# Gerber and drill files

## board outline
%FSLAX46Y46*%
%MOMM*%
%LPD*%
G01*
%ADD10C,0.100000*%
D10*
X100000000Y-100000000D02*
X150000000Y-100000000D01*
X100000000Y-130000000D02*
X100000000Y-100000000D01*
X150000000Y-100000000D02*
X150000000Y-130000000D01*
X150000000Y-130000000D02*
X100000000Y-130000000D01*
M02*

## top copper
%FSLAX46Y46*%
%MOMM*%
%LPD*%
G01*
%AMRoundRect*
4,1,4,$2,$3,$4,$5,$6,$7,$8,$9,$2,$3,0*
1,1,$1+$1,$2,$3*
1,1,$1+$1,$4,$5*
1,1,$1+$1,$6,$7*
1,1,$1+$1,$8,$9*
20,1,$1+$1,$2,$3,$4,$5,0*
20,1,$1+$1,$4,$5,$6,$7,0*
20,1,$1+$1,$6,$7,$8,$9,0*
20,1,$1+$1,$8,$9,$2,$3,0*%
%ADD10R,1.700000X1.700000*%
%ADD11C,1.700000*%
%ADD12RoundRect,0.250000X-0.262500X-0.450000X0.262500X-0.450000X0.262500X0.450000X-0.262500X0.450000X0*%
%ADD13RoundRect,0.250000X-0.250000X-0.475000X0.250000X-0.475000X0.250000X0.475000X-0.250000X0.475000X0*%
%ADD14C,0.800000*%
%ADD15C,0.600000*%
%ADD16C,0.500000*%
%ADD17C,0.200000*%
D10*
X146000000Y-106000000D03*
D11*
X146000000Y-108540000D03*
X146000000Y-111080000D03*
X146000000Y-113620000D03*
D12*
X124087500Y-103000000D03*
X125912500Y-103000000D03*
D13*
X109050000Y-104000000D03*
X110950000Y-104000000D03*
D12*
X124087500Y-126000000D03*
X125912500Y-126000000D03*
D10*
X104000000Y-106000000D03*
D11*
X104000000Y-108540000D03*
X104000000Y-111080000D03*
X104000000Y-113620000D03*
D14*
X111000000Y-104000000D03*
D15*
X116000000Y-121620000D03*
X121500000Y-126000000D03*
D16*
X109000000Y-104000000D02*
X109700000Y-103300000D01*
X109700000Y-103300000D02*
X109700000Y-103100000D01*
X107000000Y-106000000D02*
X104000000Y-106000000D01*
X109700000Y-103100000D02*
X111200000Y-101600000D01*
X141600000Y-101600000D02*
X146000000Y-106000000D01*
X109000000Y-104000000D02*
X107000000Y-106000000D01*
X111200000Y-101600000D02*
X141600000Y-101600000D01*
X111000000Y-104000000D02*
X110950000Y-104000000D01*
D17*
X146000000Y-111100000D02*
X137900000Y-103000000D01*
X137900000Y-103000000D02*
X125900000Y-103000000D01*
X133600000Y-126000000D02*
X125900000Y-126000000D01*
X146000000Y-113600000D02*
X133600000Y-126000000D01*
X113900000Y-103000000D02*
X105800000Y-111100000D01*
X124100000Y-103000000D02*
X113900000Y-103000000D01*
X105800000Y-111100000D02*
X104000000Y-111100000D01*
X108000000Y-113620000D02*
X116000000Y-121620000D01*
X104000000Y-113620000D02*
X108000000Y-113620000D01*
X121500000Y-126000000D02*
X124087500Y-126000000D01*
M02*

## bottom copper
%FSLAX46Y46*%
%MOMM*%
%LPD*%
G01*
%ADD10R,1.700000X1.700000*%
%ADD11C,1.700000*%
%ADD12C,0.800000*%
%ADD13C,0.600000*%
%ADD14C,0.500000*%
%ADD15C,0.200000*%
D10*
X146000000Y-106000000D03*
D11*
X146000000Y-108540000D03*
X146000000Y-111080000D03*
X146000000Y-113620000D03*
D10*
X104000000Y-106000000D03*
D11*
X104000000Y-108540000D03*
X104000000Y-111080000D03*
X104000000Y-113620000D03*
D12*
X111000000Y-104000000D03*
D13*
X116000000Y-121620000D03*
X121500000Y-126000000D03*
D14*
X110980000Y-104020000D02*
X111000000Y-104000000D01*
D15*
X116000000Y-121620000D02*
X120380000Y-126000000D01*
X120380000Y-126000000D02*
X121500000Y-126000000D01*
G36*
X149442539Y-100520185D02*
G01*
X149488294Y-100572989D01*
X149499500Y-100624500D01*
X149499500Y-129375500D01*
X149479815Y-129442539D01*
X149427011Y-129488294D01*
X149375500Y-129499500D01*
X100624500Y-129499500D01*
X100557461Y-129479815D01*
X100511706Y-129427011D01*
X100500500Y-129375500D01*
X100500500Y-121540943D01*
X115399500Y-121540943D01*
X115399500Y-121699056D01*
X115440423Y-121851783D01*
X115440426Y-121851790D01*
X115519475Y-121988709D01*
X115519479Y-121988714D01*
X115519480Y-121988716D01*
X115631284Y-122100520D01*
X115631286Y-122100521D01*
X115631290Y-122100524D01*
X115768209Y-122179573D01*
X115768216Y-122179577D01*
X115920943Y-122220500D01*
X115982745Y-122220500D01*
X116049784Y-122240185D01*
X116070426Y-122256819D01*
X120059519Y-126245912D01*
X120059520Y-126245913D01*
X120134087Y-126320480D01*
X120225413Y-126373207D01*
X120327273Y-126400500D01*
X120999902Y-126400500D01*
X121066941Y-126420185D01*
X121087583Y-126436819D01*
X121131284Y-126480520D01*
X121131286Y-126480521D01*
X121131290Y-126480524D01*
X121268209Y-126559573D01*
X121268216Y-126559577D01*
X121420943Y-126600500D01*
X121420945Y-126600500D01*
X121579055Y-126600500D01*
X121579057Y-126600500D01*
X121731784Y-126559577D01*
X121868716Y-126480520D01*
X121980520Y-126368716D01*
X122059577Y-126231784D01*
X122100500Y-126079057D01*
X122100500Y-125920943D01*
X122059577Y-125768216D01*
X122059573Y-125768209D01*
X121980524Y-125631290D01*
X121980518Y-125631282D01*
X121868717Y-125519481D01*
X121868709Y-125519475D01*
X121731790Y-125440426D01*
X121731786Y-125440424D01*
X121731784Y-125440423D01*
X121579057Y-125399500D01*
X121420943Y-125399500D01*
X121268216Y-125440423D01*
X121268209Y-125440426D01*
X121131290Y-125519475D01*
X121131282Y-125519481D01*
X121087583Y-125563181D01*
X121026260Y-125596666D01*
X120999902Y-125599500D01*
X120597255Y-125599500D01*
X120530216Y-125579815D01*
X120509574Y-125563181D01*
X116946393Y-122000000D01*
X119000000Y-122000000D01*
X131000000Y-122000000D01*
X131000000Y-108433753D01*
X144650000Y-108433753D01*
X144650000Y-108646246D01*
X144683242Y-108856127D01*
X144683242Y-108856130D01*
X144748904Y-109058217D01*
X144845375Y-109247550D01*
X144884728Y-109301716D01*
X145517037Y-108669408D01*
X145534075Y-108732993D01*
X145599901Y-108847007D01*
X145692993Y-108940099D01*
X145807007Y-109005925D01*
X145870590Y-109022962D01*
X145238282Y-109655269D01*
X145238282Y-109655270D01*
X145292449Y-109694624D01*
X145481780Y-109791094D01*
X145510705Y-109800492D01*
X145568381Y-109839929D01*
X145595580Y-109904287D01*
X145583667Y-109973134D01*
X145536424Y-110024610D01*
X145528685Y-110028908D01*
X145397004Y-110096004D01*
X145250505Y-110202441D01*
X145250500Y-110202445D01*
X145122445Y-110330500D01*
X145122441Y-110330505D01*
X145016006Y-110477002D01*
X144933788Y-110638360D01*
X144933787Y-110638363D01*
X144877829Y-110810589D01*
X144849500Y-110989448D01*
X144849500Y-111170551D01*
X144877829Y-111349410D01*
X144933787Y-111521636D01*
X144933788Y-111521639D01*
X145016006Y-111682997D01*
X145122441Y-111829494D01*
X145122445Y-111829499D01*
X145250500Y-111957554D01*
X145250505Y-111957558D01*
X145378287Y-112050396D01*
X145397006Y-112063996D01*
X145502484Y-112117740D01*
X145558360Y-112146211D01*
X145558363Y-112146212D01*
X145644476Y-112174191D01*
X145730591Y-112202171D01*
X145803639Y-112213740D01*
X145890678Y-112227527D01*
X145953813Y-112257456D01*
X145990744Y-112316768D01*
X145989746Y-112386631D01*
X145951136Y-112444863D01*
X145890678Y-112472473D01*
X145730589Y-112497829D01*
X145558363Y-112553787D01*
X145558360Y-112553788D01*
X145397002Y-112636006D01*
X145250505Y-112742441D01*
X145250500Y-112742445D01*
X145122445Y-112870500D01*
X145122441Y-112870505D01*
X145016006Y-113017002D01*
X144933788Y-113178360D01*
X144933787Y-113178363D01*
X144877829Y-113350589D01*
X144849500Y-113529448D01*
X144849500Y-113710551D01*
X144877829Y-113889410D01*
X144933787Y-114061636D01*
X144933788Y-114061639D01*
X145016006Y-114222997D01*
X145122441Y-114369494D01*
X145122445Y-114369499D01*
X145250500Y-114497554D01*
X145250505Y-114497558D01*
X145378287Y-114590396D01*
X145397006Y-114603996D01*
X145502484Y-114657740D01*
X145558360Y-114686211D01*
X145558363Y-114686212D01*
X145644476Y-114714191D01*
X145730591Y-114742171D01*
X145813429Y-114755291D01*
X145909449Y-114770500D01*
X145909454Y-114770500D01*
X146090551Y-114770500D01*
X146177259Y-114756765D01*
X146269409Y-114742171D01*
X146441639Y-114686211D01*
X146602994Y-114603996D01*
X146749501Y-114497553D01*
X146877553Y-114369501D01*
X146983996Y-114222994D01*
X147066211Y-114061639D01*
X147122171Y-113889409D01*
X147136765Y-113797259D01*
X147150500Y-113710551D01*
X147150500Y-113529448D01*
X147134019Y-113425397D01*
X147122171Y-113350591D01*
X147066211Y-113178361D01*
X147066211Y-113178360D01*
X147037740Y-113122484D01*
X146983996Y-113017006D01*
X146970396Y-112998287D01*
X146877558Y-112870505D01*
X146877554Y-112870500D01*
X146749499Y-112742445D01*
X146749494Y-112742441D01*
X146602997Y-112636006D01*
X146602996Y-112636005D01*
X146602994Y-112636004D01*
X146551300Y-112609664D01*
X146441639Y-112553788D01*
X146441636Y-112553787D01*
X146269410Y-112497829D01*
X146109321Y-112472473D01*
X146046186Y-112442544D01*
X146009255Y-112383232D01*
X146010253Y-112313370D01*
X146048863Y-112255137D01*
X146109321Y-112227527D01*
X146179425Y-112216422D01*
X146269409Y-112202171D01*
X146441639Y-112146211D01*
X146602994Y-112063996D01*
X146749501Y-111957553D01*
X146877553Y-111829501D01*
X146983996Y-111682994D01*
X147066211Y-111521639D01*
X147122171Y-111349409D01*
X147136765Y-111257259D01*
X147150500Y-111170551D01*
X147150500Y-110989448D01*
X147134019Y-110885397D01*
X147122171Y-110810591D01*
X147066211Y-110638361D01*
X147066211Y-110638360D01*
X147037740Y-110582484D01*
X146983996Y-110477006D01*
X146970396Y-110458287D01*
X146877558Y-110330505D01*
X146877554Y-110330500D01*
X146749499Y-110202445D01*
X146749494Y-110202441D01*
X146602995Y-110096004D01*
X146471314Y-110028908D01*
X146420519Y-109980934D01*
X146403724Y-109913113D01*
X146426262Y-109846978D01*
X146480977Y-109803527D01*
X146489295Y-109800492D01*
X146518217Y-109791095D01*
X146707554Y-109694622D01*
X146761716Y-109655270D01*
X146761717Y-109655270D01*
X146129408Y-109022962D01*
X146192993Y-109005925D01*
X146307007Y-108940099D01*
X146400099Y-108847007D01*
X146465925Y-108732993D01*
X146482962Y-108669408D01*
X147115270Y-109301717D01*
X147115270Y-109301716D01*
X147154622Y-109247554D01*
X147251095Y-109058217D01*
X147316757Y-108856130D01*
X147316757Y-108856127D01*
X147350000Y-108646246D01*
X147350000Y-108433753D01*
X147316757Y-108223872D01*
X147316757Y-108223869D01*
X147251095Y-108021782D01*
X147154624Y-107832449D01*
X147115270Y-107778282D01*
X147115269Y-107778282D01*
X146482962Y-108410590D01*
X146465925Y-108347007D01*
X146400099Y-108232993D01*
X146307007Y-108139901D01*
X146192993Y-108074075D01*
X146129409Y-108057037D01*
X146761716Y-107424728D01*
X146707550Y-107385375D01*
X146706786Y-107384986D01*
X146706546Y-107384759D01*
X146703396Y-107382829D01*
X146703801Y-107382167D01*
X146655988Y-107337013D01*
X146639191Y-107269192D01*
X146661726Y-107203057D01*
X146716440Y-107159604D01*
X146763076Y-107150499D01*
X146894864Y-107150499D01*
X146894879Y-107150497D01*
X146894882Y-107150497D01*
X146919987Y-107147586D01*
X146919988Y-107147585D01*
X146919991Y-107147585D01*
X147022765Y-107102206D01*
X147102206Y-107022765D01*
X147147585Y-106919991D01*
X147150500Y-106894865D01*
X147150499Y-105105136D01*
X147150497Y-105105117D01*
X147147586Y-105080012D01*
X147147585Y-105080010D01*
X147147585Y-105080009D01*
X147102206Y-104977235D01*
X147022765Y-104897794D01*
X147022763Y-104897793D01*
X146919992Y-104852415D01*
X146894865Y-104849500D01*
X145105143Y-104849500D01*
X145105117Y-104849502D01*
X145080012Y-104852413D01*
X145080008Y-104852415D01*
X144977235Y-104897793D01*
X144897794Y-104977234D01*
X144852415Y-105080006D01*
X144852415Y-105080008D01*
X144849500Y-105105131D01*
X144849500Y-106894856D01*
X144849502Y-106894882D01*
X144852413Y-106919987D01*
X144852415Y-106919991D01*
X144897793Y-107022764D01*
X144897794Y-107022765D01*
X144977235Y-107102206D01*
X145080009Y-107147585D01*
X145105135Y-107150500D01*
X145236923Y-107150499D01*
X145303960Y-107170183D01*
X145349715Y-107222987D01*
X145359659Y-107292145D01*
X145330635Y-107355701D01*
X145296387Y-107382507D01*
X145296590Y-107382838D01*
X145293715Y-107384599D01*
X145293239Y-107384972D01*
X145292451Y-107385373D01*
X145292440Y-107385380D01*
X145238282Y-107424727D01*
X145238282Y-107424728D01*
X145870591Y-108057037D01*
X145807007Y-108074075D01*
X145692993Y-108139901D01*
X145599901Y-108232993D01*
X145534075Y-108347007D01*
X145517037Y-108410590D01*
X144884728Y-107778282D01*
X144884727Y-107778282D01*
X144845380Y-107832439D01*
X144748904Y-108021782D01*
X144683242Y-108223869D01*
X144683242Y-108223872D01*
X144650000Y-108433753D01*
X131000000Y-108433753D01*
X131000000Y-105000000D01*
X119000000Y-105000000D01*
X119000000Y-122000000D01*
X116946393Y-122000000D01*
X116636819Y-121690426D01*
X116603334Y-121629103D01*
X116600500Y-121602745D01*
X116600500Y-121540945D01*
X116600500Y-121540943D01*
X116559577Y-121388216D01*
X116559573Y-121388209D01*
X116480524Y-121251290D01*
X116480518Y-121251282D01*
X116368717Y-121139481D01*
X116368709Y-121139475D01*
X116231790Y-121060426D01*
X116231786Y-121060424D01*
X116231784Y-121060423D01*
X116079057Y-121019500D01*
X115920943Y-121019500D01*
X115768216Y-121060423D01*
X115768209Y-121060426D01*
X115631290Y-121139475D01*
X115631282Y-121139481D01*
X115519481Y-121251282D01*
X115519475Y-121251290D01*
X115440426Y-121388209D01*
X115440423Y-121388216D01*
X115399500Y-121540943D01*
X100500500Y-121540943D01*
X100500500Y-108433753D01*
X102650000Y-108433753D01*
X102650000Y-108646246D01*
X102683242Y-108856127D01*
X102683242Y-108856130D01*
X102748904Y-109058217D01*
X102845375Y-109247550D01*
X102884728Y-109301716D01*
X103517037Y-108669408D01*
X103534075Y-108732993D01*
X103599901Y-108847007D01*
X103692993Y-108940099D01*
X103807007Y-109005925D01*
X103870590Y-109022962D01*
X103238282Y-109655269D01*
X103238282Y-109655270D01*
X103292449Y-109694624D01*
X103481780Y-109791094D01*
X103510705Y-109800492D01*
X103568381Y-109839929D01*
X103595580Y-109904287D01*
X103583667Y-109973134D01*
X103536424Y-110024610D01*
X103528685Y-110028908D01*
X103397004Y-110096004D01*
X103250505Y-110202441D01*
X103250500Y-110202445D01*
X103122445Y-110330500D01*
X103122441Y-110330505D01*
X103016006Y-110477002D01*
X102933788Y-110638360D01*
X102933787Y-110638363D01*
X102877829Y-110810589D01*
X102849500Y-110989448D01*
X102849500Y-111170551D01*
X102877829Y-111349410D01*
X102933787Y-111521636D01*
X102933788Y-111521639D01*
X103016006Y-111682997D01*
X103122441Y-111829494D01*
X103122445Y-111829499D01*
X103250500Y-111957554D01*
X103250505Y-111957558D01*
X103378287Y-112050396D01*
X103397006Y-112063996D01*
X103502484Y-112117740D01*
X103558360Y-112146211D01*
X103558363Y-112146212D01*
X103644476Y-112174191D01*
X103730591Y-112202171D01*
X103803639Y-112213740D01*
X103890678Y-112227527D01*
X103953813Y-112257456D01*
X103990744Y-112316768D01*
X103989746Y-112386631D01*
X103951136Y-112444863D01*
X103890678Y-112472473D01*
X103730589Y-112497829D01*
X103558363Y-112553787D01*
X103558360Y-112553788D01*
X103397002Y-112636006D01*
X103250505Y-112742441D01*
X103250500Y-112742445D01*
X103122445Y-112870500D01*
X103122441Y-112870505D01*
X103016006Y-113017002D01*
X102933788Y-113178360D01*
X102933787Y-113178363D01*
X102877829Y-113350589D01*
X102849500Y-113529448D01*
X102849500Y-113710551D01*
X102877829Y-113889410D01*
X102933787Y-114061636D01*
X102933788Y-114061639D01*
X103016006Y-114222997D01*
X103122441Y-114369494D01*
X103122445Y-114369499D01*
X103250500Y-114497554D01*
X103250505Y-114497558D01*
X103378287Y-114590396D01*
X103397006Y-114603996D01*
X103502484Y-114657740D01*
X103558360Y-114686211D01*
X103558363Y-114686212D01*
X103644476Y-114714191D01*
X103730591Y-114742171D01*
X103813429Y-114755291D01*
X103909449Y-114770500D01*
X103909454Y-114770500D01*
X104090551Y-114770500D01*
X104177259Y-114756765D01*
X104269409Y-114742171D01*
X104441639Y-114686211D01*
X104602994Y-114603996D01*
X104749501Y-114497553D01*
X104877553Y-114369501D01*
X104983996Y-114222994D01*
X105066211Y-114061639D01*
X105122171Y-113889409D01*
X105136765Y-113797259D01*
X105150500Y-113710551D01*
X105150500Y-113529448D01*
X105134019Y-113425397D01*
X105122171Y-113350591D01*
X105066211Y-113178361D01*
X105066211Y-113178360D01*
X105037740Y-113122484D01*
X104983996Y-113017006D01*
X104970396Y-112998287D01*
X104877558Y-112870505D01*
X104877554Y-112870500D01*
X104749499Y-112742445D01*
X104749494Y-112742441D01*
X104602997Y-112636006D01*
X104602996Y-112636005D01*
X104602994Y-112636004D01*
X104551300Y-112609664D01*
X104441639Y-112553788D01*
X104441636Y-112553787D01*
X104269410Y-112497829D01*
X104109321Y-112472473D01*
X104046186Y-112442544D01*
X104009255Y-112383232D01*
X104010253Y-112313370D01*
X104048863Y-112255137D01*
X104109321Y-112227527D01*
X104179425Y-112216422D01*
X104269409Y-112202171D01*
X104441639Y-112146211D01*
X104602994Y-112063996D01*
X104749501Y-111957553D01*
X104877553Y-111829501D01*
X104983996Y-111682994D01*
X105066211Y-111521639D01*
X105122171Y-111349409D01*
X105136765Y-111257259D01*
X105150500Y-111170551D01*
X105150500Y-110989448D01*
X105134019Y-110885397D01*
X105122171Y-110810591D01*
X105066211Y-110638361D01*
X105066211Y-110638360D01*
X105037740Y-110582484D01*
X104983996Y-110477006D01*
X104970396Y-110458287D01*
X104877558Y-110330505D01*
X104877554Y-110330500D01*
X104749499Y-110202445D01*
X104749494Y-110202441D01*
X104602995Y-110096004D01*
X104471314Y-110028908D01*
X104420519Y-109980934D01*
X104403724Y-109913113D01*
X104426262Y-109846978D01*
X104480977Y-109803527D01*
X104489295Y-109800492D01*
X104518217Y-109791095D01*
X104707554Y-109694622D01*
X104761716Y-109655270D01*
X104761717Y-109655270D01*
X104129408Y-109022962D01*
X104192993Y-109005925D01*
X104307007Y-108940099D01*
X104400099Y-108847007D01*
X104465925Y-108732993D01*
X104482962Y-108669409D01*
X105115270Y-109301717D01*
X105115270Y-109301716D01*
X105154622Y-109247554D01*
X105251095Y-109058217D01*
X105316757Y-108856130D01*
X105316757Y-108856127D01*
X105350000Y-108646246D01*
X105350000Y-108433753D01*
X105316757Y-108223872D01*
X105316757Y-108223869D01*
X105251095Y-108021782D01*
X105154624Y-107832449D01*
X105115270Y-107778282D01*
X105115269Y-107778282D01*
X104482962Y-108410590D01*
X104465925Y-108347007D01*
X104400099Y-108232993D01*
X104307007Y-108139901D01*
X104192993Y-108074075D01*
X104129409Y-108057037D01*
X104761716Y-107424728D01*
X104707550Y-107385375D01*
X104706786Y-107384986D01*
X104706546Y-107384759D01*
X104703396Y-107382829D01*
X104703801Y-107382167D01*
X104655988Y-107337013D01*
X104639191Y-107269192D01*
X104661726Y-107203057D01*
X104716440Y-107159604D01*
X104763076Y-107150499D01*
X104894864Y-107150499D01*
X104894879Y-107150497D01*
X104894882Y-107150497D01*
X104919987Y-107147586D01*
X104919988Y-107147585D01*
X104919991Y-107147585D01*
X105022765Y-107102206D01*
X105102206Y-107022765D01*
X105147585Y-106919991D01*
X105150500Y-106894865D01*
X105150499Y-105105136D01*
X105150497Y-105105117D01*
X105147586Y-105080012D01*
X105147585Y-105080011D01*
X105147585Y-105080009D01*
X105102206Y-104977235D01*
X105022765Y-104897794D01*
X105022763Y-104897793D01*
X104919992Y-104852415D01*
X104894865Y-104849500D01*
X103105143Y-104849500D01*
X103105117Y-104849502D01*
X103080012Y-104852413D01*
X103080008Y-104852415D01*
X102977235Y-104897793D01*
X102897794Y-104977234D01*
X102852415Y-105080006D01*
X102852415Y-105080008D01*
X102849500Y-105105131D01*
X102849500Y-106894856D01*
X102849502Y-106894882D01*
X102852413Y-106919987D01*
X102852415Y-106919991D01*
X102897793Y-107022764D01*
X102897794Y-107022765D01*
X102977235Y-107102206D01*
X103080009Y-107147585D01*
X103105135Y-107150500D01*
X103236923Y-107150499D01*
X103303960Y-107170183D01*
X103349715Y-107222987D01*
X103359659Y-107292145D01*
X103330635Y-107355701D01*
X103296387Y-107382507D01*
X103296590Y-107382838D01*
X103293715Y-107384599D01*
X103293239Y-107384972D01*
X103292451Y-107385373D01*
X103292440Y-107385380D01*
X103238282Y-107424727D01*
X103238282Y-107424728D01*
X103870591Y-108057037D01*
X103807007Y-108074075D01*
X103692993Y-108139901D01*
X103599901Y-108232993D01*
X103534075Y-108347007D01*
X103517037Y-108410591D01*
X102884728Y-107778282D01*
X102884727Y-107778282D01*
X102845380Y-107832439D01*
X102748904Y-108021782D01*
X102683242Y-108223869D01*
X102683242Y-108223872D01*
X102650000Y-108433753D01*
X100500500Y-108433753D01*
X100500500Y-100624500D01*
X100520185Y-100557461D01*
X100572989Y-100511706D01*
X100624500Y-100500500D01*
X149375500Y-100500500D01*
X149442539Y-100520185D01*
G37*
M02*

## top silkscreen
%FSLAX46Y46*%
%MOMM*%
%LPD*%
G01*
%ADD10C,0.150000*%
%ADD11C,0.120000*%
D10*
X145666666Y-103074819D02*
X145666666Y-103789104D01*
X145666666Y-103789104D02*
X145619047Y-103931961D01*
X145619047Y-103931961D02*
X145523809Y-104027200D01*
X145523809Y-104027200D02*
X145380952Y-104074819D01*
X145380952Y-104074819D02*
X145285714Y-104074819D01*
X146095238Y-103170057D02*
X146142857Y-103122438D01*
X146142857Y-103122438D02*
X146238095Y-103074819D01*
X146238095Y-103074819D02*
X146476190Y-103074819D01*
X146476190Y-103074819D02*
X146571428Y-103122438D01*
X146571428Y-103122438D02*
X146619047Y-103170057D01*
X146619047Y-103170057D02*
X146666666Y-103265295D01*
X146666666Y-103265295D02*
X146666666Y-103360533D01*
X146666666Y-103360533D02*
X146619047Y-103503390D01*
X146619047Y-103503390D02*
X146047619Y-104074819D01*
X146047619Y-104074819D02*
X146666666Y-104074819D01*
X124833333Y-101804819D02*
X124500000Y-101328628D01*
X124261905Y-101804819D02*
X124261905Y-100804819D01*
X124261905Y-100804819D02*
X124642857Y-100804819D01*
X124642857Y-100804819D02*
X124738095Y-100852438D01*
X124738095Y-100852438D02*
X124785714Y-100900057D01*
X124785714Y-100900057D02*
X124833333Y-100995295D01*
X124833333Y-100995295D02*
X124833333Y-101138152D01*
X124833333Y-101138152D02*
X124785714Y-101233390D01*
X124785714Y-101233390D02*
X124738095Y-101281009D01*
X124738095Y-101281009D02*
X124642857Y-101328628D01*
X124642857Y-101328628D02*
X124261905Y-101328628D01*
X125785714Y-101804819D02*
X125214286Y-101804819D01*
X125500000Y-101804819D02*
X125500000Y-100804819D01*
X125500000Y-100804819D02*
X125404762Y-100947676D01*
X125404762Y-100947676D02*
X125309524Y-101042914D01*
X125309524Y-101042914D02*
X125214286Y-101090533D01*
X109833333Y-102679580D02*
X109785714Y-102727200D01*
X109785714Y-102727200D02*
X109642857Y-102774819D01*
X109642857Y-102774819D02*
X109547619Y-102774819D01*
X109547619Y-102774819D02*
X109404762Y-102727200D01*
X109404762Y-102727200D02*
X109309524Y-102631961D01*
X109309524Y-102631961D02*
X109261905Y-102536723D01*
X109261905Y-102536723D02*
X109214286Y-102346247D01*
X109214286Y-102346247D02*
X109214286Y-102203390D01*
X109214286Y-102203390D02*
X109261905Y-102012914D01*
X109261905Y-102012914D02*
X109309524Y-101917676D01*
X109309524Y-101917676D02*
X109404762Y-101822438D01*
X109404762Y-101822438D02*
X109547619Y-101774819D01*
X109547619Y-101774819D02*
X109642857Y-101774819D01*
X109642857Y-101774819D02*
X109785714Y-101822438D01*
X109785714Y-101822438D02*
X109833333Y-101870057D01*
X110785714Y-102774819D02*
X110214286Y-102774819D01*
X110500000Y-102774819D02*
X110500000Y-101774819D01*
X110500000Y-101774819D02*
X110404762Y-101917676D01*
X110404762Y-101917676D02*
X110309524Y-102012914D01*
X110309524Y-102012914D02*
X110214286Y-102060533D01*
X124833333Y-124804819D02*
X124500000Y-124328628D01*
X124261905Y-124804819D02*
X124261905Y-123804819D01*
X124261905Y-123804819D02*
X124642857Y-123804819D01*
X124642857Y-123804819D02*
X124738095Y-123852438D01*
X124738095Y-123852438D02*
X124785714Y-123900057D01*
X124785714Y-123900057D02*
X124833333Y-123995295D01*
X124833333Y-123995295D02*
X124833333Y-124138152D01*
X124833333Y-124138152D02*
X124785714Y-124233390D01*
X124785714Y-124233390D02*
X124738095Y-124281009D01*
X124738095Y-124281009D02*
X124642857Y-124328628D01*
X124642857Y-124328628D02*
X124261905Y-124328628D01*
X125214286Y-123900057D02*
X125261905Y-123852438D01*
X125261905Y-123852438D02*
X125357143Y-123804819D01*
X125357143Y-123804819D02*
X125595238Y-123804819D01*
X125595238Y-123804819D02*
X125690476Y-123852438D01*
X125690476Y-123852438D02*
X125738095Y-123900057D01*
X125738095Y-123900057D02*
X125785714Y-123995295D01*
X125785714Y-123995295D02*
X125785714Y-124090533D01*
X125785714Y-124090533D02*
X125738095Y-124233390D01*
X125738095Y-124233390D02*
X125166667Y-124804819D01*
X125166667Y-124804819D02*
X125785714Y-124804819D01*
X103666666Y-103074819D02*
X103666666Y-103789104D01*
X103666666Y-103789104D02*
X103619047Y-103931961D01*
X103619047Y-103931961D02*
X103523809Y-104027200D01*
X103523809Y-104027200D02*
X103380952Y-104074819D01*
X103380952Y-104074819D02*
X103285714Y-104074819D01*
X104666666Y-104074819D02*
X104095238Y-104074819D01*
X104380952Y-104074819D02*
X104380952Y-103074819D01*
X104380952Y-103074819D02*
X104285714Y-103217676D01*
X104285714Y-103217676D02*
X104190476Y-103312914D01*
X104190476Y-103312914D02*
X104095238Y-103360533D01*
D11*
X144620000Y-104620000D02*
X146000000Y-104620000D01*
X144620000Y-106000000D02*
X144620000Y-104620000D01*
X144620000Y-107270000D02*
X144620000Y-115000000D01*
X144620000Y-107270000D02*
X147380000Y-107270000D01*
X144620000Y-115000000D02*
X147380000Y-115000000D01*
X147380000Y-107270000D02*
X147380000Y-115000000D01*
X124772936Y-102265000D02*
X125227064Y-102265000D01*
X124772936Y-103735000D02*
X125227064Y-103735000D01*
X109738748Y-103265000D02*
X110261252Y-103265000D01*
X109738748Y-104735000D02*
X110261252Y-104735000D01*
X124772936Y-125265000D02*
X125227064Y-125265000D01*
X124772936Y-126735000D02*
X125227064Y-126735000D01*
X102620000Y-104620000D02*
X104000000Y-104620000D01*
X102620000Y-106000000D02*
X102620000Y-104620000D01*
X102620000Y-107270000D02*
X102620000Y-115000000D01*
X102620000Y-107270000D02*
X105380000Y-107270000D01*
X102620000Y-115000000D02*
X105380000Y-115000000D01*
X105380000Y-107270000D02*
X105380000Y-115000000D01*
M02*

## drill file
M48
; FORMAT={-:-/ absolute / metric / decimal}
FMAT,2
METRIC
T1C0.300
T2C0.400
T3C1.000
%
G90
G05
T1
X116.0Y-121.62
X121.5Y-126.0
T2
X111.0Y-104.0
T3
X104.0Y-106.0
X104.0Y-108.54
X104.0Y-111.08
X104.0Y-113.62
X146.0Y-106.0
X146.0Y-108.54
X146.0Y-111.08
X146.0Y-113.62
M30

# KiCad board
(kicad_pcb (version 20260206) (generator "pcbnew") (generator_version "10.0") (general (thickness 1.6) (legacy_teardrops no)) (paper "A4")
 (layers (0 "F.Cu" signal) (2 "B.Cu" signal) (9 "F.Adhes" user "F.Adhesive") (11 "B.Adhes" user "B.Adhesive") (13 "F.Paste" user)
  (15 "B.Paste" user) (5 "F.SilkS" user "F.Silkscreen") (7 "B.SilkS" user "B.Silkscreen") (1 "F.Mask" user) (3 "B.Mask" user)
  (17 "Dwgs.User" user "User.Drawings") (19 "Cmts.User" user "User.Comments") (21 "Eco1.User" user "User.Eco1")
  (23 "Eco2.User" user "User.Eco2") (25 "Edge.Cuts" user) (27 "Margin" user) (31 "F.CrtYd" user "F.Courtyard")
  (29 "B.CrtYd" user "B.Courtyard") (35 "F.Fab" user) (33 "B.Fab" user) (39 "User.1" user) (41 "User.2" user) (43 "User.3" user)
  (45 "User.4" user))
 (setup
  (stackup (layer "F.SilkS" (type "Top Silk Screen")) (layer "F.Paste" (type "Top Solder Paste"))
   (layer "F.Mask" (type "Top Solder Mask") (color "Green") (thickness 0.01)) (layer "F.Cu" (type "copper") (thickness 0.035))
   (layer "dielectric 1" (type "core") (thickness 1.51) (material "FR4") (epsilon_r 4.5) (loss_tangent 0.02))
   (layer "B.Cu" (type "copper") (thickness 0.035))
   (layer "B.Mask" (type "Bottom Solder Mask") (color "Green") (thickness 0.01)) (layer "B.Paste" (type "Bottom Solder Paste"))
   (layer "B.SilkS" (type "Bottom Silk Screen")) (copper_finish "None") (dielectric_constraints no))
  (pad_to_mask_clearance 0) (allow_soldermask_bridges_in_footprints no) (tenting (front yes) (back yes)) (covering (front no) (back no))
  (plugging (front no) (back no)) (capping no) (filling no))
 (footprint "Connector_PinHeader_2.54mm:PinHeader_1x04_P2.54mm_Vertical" (layer "F.Cu") (at 146 106)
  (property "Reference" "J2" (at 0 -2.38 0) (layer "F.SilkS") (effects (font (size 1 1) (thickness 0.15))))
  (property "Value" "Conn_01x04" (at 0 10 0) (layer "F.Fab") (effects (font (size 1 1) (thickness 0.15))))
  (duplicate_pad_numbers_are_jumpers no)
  (fp_line (start -1.38 -1.38) (end 0 -1.38) (stroke (width 0.12) (type solid)) (layer "F.SilkS"))
  (fp_line (start -1.38 0) (end -1.38 -1.38) (stroke (width 0.12) (type solid)) (layer "F.SilkS"))
  (fp_line (start -1.38 1.27) (end -1.38 9) (stroke (width 0.12) (type solid)) (layer "F.SilkS"))
  (fp_line (start -1.38 1.27) (end 1.38 1.27) (stroke (width 0.12) (type solid)) (layer "F.SilkS"))
  (fp_line (start -1.38 9) (end 1.38 9) (stroke (width 0.12) (type solid)) (layer "F.SilkS"))
  (fp_line (start 1.38 1.27) (end 1.38 9) (stroke (width 0.12) (type solid)) (layer "F.SilkS"))
  (pad "1" thru_hole rect (at 0 0) (size 1.7 1.7) (drill 1) (layers "*.Cu" "*.Mask") (remove_unused_layers no) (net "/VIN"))
  (pad "2" thru_hole circle (at 0 2.54) (size 1.7 1.7) (drill 1) (layers "*.Cu" "*.Mask") (remove_unused_layers no) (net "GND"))
  (pad "3" thru_hole circle (at 0 5.08) (size 1.7 1.7) (drill 1) (layers "*.Cu" "*.Mask") (remove_unused_layers no) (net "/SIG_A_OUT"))
  (pad "4" thru_hole circle (at 0 7.62) (size 1.7 1.7) (drill 1) (layers "*.Cu" "*.Mask") (remove_unused_layers no) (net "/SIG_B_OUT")))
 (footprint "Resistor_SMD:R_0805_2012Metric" (layer "F.Cu") (at 125 103)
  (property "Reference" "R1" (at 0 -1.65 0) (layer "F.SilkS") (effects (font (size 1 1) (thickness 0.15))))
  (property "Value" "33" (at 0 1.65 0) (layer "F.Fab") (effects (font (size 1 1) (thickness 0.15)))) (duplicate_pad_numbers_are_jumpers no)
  (fp_line (start -0.227064 -0.735) (end 0.227064 -0.735) (stroke (width 0.12) (type solid)) (layer "F.SilkS"))
  (fp_line (start -0.227064 0.735) (end 0.227064 0.735) (stroke (width 0.12) (type solid)) (layer "F.SilkS"))
  (pad "1" smd roundrect (at -0.9125 0) (size 1.025 1.4) (layers "F.Cu" "F.Mask" "F.Paste") (roundrect_rratio 0.243902) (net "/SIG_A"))
  (pad "2" smd roundrect (at 0.9125 0) (size 1.025 1.4) (layers "F.Cu" "F.Mask" "F.Paste") (roundrect_rratio 0.243902) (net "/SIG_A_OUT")))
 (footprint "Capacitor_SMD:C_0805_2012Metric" (layer "F.Cu") (at 110 104)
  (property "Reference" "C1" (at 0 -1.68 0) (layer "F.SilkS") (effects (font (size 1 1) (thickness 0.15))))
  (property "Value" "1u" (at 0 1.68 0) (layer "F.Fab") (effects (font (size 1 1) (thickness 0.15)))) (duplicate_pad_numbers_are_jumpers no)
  (fp_line (start -0.261252 -0.735) (end 0.261252 -0.735) (stroke (width 0.12) (type solid)) (layer "F.SilkS"))
  (fp_line (start -0.261252 0.735) (end 0.261252 0.735) (stroke (width 0.12) (type solid)) (layer "F.SilkS"))
  (pad "1" smd roundrect (at -0.95 0) (size 1 1.45) (layers "F.Cu" "F.Mask" "F.Paste") (roundrect_rratio 0.25) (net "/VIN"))
  (pad "2" smd roundrect (at 0.95 0) (size 1 1.45) (layers "F.Cu" "F.Mask" "F.Paste") (roundrect_rratio 0.25) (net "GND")))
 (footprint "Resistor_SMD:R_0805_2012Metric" (layer "F.Cu") (at 125 126)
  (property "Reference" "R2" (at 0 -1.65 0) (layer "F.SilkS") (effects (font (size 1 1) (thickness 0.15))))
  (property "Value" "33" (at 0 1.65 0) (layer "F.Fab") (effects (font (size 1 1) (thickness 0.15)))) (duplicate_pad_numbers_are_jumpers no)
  (fp_line (start -0.227064 -0.735) (end 0.227064 -0.735) (stroke (width 0.12) (type solid)) (layer "F.SilkS"))
  (fp_line (start -0.227064 0.735) (end 0.227064 0.735) (stroke (width 0.12) (type solid)) (layer "F.SilkS"))
  (pad "1" smd roundrect (at -0.9125 0) (size 1.025 1.4) (layers "F.Cu" "F.Mask" "F.Paste") (roundrect_rratio 0.243902) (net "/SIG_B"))
  (pad "2" smd roundrect (at 0.9125 0) (size 1.025 1.4) (layers "F.Cu" "F.Mask" "F.Paste") (roundrect_rratio 0.243902) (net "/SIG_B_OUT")))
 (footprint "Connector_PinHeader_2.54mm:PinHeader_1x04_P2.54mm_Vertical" (layer "F.Cu") (at 104 106)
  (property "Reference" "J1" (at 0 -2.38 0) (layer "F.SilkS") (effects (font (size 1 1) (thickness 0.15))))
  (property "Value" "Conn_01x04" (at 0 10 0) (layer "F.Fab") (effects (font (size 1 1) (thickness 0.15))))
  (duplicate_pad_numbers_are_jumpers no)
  (fp_line (start -1.38 -1.38) (end 0 -1.38) (stroke (width 0.12) (type solid)) (layer "F.SilkS"))
  (fp_line (start -1.38 0) (end -1.38 -1.38) (stroke (width 0.12) (type solid)) (layer "F.SilkS"))
  (fp_line (start -1.38 1.27) (end -1.38 9) (stroke (width 0.12) (type solid)) (layer "F.SilkS"))
  (fp_line (start -1.38 1.27) (end 1.38 1.27) (stroke (width 0.12) (type solid)) (layer "F.SilkS"))
  (fp_line (start -1.38 9) (end 1.38 9) (stroke (width 0.12) (type solid)) (layer "F.SilkS"))
  (fp_line (start 1.38 1.27) (end 1.38 9) (stroke (width 0.12) (type solid)) (layer "F.SilkS"))
  (pad "1" thru_hole rect (at 0 0) (size 1.7 1.7) (drill 1) (layers "*.Cu" "*.Mask") (remove_unused_layers no) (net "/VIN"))
  (pad "2" thru_hole circle (at 0 2.54) (size 1.7 1.7) (drill 1) (layers "*.Cu" "*.Mask") (remove_unused_layers no) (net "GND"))
  (pad "3" thru_hole circle (at 0 5.08) (size 1.7 1.7) (drill 1) (layers "*.Cu" "*.Mask") (remove_unused_layers no) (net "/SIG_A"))
  (pad "4" thru_hole circle (at 0 7.62) (size 1.7 1.7) (drill 1) (layers "*.Cu" "*.Mask") (remove_unused_layers no) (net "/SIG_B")))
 (gr_line (start 100 100) (end 150 100) (stroke (width 0.1) (type default)) (layer "Edge.Cuts"))
 (gr_line (start 100 130) (end 100 100) (stroke (width 0.1) (type default)) (layer "Edge.Cuts"))
 (gr_line (start 150 100) (end 150 130) (stroke (width 0.1) (type default)) (layer "Edge.Cuts"))
 (gr_line (start 150 130) (end 100 130) (stroke (width 0.1) (type default)) (layer "Edge.Cuts"))
 (segment (start 109 104) (end 109.7 103.3) (width 0.5) (layer "F.Cu") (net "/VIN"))
 (segment (start 109.7 103.3) (end 109.7 103.1) (width 0.5) (layer "F.Cu") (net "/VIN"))
 (segment (start 107 106) (end 104 106) (width 0.5) (layer "F.Cu") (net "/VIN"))
 (segment (start 109.7 103.1) (end 111.2 101.6) (width 0.5) (layer "F.Cu") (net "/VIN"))
 (segment (start 141.6 101.6) (end 146 106) (width 0.5) (layer "F.Cu") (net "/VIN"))
 (segment (start 109 104) (end 107 106) (width 0.5) (layer "F.Cu") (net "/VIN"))
 (segment (start 111.2 101.6) (end 141.6 101.6) (width 0.5) (layer "F.Cu") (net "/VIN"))
 (segment (start 111 104) (end 110.95 104) (width 0.5) (layer "F.Cu") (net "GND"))
 (via (at 111 104) (size 0.8) (drill 0.4) (layers "F.Cu" "B.Cu") (capping yes) (filling yes) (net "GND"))
 (segment (start 110.98 104.02) (end 111 104) (width 0.5) (layer "B.Cu") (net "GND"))
 (segment (start 146 111.1) (end 137.9 103) (width 0.2) (layer "F.Cu") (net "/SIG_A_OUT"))
 (segment (start 137.9 103) (end 125.9 103) (width 0.2) (layer "F.Cu") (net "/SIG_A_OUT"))
 (segment (start 133.6 126) (end 125.9 126) (width 0.2) (layer "F.Cu") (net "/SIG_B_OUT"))
 (segment (start 146 113.6) (end 133.6 126) (width 0.2) (layer "F.Cu") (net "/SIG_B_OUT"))
 (segment (start 113.9 103) (end 105.8 111.1) (width 0.2) (layer "F.Cu") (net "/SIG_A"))
 (segment (start 124.1 103) (end 113.9 103) (width 0.2) (layer "F.Cu") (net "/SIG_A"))
 (segment (start 105.8 111.1) (end 104 111.1) (width 0.2) (layer "F.Cu") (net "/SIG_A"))
 (segment (start 108 113.62) (end 116 121.62) (width 0.2) (locked yes) (layer "F.Cu") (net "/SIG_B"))
 (segment (start 104 113.62) (end 108 113.62) (width 0.2) (locked yes) (layer "F.Cu") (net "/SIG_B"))
 (segment (start 121.5 126) (end 124.0875 126) (width 0.2) (locked yes) (layer "F.Cu") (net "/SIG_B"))
 (via (at 116 121.62) (size 0.6) (drill 0.3) (layers "F.Cu" "B.Cu") (locked yes) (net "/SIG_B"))
 (via (at 121.5 126) (size 0.6) (drill 0.3) (layers "F.Cu" "B.Cu") (locked yes) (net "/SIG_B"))
 (segment (start 116 121.62) (end 120.38 126) (width 0.2) (locked yes) (layer "B.Cu") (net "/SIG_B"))
 (segment (start 120.38 126) (end 121.5 126) (width 0.2) (locked yes) (layer "B.Cu") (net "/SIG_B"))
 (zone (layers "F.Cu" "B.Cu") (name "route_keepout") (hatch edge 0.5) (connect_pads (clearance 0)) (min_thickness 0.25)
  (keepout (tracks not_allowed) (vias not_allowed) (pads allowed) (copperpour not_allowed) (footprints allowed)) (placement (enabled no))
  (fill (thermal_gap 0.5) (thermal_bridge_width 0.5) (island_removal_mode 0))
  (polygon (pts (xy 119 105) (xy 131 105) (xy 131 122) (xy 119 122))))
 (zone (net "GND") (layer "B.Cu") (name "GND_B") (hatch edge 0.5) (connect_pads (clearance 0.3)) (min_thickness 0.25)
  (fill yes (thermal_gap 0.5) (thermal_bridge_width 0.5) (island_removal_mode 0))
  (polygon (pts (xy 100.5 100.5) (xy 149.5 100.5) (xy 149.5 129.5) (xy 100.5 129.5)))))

